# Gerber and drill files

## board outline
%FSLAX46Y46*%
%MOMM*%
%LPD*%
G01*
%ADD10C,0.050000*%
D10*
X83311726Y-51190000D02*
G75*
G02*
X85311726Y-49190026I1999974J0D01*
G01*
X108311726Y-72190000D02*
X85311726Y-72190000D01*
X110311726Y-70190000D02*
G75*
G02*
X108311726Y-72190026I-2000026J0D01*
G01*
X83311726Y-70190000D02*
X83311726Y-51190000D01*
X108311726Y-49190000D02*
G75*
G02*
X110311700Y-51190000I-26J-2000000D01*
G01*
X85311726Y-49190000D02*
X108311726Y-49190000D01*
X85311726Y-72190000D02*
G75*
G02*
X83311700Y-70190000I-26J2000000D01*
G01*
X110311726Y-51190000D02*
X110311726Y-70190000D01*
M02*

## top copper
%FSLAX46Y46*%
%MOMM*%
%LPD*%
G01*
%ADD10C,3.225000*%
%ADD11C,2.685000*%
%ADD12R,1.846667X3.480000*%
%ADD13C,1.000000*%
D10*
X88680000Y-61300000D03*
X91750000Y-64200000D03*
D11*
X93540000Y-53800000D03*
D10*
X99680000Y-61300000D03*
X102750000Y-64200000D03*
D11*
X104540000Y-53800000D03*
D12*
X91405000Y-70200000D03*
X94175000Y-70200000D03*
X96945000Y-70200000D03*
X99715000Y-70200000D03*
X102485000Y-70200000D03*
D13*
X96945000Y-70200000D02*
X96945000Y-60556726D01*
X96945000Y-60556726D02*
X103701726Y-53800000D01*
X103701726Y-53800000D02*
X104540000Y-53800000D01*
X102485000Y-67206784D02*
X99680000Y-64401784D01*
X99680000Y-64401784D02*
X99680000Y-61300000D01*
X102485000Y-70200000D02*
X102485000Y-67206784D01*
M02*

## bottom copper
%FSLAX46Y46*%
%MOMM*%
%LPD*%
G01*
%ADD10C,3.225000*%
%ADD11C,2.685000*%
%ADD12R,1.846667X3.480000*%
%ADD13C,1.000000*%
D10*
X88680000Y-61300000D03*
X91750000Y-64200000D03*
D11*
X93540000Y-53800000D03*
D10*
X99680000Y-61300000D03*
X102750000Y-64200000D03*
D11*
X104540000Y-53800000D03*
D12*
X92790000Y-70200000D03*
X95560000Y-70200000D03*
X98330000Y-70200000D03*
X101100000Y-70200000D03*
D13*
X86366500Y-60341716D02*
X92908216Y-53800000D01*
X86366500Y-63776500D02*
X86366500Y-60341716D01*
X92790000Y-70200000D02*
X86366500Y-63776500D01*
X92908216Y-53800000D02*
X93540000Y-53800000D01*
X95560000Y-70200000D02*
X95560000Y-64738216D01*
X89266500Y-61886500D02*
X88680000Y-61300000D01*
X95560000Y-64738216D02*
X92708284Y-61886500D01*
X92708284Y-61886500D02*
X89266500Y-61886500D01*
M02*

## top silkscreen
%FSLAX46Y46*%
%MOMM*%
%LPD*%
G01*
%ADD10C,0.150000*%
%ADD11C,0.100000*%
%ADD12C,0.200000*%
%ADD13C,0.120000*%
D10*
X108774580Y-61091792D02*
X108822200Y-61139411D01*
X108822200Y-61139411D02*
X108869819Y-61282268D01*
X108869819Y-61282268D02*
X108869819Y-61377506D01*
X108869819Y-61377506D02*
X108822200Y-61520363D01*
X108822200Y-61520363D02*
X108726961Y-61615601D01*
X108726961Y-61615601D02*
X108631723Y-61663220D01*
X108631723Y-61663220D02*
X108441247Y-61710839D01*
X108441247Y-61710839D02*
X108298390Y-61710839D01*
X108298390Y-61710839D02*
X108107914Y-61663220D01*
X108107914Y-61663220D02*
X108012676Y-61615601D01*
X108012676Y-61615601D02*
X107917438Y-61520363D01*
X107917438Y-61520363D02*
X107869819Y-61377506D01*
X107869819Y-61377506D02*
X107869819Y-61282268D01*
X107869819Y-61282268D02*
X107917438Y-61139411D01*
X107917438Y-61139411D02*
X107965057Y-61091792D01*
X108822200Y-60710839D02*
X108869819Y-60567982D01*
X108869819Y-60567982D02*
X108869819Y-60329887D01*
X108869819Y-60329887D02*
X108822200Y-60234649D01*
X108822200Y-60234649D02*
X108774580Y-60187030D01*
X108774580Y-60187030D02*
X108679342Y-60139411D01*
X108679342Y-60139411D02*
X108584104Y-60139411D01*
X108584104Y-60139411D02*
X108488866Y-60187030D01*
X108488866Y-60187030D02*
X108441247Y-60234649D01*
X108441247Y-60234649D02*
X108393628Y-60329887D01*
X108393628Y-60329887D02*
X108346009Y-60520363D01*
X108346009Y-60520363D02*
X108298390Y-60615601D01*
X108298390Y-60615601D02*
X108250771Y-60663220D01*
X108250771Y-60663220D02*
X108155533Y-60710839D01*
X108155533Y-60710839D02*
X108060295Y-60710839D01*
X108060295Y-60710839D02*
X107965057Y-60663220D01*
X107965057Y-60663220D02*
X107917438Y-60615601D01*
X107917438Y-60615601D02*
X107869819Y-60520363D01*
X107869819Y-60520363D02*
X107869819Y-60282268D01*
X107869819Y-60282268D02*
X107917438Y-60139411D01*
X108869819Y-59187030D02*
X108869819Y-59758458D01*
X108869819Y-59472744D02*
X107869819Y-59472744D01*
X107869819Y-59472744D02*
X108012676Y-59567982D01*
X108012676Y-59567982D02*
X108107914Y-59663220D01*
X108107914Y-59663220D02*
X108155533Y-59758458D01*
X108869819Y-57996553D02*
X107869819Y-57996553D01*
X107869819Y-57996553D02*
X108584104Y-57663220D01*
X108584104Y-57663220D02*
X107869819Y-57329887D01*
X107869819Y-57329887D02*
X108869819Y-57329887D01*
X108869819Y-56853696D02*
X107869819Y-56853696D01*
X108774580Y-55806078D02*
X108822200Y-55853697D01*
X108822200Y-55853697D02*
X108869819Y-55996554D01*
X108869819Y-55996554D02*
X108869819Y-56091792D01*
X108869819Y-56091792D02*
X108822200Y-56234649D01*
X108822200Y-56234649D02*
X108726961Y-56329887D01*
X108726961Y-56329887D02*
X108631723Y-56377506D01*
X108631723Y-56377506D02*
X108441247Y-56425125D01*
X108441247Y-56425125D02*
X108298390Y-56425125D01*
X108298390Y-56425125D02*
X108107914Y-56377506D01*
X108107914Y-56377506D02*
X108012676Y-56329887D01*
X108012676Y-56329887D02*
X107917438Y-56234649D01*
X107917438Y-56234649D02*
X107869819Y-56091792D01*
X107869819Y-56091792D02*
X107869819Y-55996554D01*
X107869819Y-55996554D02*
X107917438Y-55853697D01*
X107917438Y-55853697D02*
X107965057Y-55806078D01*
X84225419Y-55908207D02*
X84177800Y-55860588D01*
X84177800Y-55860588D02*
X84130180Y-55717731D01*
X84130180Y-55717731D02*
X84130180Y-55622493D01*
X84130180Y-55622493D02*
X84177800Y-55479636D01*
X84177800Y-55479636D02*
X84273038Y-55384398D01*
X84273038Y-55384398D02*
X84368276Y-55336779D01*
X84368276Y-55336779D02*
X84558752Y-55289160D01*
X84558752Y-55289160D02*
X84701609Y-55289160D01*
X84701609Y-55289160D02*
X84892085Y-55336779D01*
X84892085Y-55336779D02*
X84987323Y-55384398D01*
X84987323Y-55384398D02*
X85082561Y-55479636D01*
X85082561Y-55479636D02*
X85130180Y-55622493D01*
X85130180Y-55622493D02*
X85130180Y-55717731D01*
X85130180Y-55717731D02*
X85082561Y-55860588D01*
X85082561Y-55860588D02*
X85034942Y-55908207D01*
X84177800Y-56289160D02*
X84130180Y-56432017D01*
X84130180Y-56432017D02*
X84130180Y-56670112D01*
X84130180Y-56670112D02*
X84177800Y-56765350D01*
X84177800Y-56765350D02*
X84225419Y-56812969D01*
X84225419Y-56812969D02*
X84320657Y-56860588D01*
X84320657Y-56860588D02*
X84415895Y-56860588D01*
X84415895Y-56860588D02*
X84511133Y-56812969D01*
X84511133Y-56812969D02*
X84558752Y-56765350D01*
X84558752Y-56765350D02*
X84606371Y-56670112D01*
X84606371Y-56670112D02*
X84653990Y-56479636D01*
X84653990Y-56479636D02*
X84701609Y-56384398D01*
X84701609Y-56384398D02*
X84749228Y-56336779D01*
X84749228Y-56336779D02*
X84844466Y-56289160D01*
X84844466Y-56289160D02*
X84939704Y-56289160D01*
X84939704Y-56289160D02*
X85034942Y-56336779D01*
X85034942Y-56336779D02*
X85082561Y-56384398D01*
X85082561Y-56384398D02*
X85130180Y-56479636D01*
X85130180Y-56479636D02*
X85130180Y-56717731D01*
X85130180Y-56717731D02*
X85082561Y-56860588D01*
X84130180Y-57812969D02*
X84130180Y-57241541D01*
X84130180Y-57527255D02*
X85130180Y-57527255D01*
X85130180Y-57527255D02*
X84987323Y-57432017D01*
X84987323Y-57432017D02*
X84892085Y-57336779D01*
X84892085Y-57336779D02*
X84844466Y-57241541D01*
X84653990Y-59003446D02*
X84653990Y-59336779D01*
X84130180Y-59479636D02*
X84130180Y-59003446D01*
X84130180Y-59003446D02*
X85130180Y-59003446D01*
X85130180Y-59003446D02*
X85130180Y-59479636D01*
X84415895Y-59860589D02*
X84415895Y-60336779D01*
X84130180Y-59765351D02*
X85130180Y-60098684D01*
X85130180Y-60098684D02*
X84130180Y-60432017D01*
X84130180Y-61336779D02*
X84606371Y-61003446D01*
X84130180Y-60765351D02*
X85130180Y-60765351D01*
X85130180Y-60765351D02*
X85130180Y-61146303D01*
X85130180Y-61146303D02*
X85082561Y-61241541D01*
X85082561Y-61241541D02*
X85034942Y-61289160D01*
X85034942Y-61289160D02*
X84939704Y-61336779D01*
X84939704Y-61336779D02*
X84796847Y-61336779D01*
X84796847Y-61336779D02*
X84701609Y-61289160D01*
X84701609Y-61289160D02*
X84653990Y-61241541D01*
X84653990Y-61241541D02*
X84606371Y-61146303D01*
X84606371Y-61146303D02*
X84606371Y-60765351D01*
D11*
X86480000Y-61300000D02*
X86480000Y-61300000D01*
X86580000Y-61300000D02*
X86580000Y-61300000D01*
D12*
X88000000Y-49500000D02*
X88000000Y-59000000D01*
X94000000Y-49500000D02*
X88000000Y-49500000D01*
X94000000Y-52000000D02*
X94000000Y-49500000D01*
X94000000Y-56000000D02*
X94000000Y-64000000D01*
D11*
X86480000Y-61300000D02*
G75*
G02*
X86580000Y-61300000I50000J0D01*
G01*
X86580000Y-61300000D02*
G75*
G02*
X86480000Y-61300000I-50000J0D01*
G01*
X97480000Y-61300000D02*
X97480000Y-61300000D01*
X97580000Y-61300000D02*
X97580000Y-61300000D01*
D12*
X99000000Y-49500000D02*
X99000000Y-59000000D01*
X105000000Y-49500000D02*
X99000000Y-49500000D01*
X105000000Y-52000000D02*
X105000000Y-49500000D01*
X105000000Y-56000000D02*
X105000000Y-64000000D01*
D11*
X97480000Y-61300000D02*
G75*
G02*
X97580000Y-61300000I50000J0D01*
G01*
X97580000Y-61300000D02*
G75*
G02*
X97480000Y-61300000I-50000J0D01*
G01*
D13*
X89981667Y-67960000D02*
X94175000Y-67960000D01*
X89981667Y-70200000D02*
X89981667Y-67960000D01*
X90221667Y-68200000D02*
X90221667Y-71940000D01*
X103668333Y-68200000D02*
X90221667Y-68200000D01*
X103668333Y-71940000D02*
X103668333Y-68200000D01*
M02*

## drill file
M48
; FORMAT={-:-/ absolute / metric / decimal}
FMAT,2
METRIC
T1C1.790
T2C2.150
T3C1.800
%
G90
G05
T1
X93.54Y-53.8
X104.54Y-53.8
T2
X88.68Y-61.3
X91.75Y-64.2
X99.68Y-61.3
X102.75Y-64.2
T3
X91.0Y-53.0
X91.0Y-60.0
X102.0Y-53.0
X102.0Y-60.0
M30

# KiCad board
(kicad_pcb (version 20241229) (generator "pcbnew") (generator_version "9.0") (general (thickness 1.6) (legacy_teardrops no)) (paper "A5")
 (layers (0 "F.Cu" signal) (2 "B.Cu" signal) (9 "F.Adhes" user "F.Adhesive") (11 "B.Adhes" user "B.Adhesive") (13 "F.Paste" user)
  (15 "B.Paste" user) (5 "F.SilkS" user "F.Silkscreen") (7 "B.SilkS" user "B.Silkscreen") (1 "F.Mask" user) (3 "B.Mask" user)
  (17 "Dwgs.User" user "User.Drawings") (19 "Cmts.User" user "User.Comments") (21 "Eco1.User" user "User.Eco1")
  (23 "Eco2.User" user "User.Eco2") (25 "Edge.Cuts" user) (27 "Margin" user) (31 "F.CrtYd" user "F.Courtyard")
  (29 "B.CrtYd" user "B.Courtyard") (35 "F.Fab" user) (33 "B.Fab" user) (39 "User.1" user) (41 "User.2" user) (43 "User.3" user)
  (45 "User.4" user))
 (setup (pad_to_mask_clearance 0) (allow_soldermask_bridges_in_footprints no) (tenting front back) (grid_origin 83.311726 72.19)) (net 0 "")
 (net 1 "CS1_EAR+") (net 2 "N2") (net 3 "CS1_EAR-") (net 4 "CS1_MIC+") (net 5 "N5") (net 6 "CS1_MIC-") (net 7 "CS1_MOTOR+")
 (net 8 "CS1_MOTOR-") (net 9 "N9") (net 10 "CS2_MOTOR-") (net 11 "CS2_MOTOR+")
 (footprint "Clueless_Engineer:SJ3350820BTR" (layer "F.Cu") (at 88.68 61.3 -90)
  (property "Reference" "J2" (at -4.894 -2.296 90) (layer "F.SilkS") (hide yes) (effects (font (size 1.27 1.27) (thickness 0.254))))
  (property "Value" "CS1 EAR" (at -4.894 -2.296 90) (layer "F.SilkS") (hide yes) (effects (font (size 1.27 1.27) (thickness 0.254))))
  (fp_line (start 0 2.2) (end 0 2.2) (stroke (width 0.1) (type solid)) (layer "F.SilkS"))
  (fp_line (start 0 2.1) (end 0 2.1) (stroke (width 0.1) (type solid)) (layer "F.SilkS"))
  (fp_line (start -11.8 0.68) (end -2.3 0.68) (stroke (width 0.2) (type solid)) (layer "F.SilkS"))
  (fp_line (start -11.8 -5.32) (end -11.8 0.68) (stroke (width 0.2) (type solid)) (layer "F.SilkS"))
  (fp_line (start -9.3 -5.32) (end -11.8 -5.32) (stroke (width 0.2) (type solid)) (layer "F.SilkS"))
  (fp_line (start -5.3 -5.32) (end 2.7 -5.32) (stroke (width 0.2) (type solid)) (layer "F.SilkS"))
  (fp_arc (start 0 2.2) (mid -0.05 2.15) (end 0 2.1) (stroke (width 0.1) (type solid)) (layer "F.SilkS"))
  (fp_arc (start 0 2.1) (mid 0.05 2.15) (end 0 2.2) (stroke (width 0.1) (type solid)) (layer "F.SilkS"))
  (pad "" np_thru_hole circle (at -8.3 -2.32 270) (size 1.8 1.8) (drill 1.8) (layers "*.Cu" "*.Mask"))
  (pad "" np_thru_hole circle (at -1.3 -2.32 270) (size 1.8 1.8) (drill 1.8) (layers "*.Cu" "*.Mask"))
  (pad "2" thru_hole circle (at 0 0 270) (size 3.225 3.225) (drill 2.15) (layers "*.Cu" "*.Mask") (remove_unused_layers no)
   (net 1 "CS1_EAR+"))
  (pad "3" thru_hole circle (at 2.9 -3.07 270) (size 3.225 3.225) (drill 2.15) (layers "*.Cu" "*.Mask") (remove_unused_layers no)
   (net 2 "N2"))
  (pad "5" thru_hole circle (at -7.5 -4.86 270) (size 2.685 2.685) (drill 1.79) (layers "*.Cu" "*.Mask") (remove_unused_layers no)
   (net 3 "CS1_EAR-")))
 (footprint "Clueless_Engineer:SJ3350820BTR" (layer "F.Cu") (at 99.68 61.3 -90)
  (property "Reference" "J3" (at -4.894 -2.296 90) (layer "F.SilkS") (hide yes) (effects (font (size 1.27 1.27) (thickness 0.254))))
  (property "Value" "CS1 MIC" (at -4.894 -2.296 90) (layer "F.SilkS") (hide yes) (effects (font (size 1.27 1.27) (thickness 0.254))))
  (fp_line (start 0 2.2) (end 0 2.2) (stroke (width 0.1) (type solid)) (layer "F.SilkS"))
  (fp_line (start 0 2.1) (end 0 2.1) (stroke (width 0.1) (type solid)) (layer "F.SilkS"))
  (fp_line (start -11.8 0.68) (end -2.3 0.68) (stroke (width 0.2) (type solid)) (layer "F.SilkS"))
  (fp_line (start -11.8 -5.32) (end -11.8 0.68) (stroke (width 0.2) (type solid)) (layer "F.SilkS"))
  (fp_line (start -9.3 -5.32) (end -11.8 -5.32) (stroke (width 0.2) (type solid)) (layer "F.SilkS"))
  (fp_line (start -5.3 -5.32) (end 2.7 -5.32) (stroke (width 0.2) (type solid)) (layer "F.SilkS"))
  (fp_arc (start 0 2.2) (mid -0.05 2.15) (end 0 2.1) (stroke (width 0.1) (type solid)) (layer "F.SilkS"))
  (fp_arc (start 0 2.1) (mid 0.05 2.15) (end 0 2.2) (stroke (width 0.1) (type solid)) (layer "F.SilkS"))
  (pad "" np_thru_hole circle (at -8.3 -2.32 270) (size 1.8 1.8) (drill 1.8) (layers "*.Cu" "*.Mask"))
  (pad "" np_thru_hole circle (at -1.3 -2.32 270) (size 1.8 1.8) (drill 1.8) (layers "*.Cu" "*.Mask"))
  (pad "2" thru_hole circle (at 0 0 270) (size 3.225 3.225) (drill 2.15) (layers "*.Cu" "*.Mask") (remove_unused_layers no)
   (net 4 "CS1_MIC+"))
  (pad "3" thru_hole circle (at 2.9 -3.07 270) (size 3.225 3.225) (drill 2.15) (layers "*.Cu" "*.Mask") (remove_unused_layers no)
   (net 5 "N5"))
  (pad "5" thru_hole circle (at -7.5 -4.86 270) (size 2.685 2.685) (drill 1.79) (layers "*.Cu" "*.Mask") (remove_unused_layers no)
   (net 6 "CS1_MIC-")))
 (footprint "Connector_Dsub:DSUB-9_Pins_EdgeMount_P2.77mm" (layer "F.Cu") (at 96.945 70.2)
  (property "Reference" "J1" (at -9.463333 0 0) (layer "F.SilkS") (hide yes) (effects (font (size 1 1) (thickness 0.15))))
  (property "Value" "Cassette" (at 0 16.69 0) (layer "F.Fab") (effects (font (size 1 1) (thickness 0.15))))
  (fp_line (start -6.963333 -2.24) (end -2.77 -2.24) (stroke (width 0.12) (type solid)) (layer "F.SilkS"))
  (fp_line (start -6.963333 0) (end -6.963333 -2.24) (stroke (width 0.12) (type solid)) (layer "F.SilkS"))
  (fp_line (start -6.723333 -2) (end -6.723333 1.74) (stroke (width 0.12) (type solid)) (layer "F.SilkS"))
  (fp_line (start 6.723333 -2) (end -6.723333 -2) (stroke (width 0.12) (type solid)) (layer "F.SilkS"))
  (fp_line (start 6.723333 1.74) (end 6.723333 -2) (stroke (width 0.12) (type solid)) (layer "F.SilkS"))
  (pad "1" smd rect (at -5.54 0) (size 1.846667 3.48) (layers "F.Cu" "F.Mask" "F.Paste") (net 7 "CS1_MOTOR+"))
  (pad "2" smd rect (at -2.77 0) (size 1.846667 3.48) (layers "F.Cu" "F.Mask" "F.Paste") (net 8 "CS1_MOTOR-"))
  (pad "3" smd rect (at 0 0) (size 1.846667 3.48) (layers "F.Cu" "F.Mask" "F.Paste") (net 6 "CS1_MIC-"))
  (pad "4" smd rect (at 2.77 0) (size 1.846667 3.48) (layers "F.Cu" "F.Mask" "F.Paste") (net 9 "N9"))
  (pad "5" smd rect (at 5.54 0) (size 1.846667 3.48) (layers "F.Cu" "F.Mask" "F.Paste") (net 4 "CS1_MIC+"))
  (pad "6" smd rect (at -4.155 0) (size 1.846667 3.48) (layers "B.Cu" "B.Mask" "B.Paste") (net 3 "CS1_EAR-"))
  (pad "7" smd rect (at -1.385 0) (size 1.846667 3.48) (layers "B.Cu" "B.Mask" "B.Paste") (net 1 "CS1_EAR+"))
  (pad "8" smd rect (at 1.385 0) (size 1.846667 3.48) (layers "B.Cu" "B.Mask" "B.Paste") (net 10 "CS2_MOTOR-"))
  (pad "9" smd rect (at 4.155 0) (size 1.846667 3.48) (layers "B.Cu" "B.Mask" "B.Paste") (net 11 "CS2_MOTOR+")))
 (gr_arc (start 83.311726 51.19) (mid 83.897514 49.775796) (end 85.311726 49.19) (stroke (width 0.05) (type default)) (layer "Edge.Cuts"))
 (gr_line (start 108.311726 72.19) (end 85.311726 72.19) (stroke (width 0.05) (type default)) (layer "Edge.Cuts"))
 (gr_arc (start 110.311726 70.19) (mid 109.72594 71.604214) (end 108.311726 72.19) (stroke (width 0.05) (type default)) (layer "Edge.Cuts"))
 (gr_line (start 83.311726 70.19) (end 83.311726 51.19) (stroke (width 0.05) (type default)) (layer "Edge.Cuts"))
 (gr_arc (start 108.311726 49.19) (mid 109.72594 49.775786) (end 110.311726 51.19) (stroke (width 0.05) (type default)) (layer "Edge.Cuts"))
 (gr_line (start 85.311726 49.19) (end 108.311726 49.19) (stroke (width 0.05) (type default)) (layer "Edge.Cuts"))
 (gr_arc (start 85.311726 72.19) (mid 83.897512 71.604214) (end 83.311726 70.19) (stroke (width 0.05) (type default)) (layer "Edge.Cuts"))
 (gr_line (start 110.311726 51.19) (end 110.311726 70.19) (stroke (width 0.05) (type default)) (layer "Edge.Cuts"))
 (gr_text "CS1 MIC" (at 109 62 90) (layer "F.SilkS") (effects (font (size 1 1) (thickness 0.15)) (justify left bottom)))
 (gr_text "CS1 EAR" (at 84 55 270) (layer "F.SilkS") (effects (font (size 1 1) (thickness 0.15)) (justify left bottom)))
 (segment (start 96.945 70.2) (end 96.945 60.556726) (width 1) (layer "F.Cu") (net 6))
 (segment (start 96.945 60.556726) (end 103.701726 53.8) (width 1) (layer "F.Cu") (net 6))
 (segment (start 103.701726 53.8) (end 104.54 53.8) (width 1) (layer "F.Cu") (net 6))
 (segment (start 102.485 67.206784) (end 99.68 64.401784) (width 1) (layer "F.Cu") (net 4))
 (segment (start 99.68 64.401784) (end 99.68 61.3) (width 1) (layer "F.Cu") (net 4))
 (segment (start 102.485 70.2) (end 102.485 67.206784) (width 1) (layer "F.Cu") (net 4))
 (segment (start 86.3665 60.341716) (end 92.908216 53.8) (width 1) (layer "B.Cu") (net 3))
 (segment (start 86.3665 63.7765) (end 86.3665 60.341716) (width 1) (layer "B.Cu") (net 3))
 (segment (start 92.79 70.2) (end 86.3665 63.7765) (width 1) (layer "B.Cu") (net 3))
 (segment (start 92.908216 53.8) (end 93.54 53.8) (width 1) (layer "B.Cu") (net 3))
 (segment (start 95.56 70.2) (end 95.56 64.738216) (width 1) (layer "B.Cu") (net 1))
 (segment (start 89.2665 61.8865) (end 88.68 61.3) (width 1) (layer "B.Cu") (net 1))
 (segment (start 95.56 64.738216) (end 92.708284 61.8865) (width 1) (layer "B.Cu") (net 1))
 (segment (start 92.708284 61.8865) (end 89.2665 61.8865) (width 1) (layer "B.Cu") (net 1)))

